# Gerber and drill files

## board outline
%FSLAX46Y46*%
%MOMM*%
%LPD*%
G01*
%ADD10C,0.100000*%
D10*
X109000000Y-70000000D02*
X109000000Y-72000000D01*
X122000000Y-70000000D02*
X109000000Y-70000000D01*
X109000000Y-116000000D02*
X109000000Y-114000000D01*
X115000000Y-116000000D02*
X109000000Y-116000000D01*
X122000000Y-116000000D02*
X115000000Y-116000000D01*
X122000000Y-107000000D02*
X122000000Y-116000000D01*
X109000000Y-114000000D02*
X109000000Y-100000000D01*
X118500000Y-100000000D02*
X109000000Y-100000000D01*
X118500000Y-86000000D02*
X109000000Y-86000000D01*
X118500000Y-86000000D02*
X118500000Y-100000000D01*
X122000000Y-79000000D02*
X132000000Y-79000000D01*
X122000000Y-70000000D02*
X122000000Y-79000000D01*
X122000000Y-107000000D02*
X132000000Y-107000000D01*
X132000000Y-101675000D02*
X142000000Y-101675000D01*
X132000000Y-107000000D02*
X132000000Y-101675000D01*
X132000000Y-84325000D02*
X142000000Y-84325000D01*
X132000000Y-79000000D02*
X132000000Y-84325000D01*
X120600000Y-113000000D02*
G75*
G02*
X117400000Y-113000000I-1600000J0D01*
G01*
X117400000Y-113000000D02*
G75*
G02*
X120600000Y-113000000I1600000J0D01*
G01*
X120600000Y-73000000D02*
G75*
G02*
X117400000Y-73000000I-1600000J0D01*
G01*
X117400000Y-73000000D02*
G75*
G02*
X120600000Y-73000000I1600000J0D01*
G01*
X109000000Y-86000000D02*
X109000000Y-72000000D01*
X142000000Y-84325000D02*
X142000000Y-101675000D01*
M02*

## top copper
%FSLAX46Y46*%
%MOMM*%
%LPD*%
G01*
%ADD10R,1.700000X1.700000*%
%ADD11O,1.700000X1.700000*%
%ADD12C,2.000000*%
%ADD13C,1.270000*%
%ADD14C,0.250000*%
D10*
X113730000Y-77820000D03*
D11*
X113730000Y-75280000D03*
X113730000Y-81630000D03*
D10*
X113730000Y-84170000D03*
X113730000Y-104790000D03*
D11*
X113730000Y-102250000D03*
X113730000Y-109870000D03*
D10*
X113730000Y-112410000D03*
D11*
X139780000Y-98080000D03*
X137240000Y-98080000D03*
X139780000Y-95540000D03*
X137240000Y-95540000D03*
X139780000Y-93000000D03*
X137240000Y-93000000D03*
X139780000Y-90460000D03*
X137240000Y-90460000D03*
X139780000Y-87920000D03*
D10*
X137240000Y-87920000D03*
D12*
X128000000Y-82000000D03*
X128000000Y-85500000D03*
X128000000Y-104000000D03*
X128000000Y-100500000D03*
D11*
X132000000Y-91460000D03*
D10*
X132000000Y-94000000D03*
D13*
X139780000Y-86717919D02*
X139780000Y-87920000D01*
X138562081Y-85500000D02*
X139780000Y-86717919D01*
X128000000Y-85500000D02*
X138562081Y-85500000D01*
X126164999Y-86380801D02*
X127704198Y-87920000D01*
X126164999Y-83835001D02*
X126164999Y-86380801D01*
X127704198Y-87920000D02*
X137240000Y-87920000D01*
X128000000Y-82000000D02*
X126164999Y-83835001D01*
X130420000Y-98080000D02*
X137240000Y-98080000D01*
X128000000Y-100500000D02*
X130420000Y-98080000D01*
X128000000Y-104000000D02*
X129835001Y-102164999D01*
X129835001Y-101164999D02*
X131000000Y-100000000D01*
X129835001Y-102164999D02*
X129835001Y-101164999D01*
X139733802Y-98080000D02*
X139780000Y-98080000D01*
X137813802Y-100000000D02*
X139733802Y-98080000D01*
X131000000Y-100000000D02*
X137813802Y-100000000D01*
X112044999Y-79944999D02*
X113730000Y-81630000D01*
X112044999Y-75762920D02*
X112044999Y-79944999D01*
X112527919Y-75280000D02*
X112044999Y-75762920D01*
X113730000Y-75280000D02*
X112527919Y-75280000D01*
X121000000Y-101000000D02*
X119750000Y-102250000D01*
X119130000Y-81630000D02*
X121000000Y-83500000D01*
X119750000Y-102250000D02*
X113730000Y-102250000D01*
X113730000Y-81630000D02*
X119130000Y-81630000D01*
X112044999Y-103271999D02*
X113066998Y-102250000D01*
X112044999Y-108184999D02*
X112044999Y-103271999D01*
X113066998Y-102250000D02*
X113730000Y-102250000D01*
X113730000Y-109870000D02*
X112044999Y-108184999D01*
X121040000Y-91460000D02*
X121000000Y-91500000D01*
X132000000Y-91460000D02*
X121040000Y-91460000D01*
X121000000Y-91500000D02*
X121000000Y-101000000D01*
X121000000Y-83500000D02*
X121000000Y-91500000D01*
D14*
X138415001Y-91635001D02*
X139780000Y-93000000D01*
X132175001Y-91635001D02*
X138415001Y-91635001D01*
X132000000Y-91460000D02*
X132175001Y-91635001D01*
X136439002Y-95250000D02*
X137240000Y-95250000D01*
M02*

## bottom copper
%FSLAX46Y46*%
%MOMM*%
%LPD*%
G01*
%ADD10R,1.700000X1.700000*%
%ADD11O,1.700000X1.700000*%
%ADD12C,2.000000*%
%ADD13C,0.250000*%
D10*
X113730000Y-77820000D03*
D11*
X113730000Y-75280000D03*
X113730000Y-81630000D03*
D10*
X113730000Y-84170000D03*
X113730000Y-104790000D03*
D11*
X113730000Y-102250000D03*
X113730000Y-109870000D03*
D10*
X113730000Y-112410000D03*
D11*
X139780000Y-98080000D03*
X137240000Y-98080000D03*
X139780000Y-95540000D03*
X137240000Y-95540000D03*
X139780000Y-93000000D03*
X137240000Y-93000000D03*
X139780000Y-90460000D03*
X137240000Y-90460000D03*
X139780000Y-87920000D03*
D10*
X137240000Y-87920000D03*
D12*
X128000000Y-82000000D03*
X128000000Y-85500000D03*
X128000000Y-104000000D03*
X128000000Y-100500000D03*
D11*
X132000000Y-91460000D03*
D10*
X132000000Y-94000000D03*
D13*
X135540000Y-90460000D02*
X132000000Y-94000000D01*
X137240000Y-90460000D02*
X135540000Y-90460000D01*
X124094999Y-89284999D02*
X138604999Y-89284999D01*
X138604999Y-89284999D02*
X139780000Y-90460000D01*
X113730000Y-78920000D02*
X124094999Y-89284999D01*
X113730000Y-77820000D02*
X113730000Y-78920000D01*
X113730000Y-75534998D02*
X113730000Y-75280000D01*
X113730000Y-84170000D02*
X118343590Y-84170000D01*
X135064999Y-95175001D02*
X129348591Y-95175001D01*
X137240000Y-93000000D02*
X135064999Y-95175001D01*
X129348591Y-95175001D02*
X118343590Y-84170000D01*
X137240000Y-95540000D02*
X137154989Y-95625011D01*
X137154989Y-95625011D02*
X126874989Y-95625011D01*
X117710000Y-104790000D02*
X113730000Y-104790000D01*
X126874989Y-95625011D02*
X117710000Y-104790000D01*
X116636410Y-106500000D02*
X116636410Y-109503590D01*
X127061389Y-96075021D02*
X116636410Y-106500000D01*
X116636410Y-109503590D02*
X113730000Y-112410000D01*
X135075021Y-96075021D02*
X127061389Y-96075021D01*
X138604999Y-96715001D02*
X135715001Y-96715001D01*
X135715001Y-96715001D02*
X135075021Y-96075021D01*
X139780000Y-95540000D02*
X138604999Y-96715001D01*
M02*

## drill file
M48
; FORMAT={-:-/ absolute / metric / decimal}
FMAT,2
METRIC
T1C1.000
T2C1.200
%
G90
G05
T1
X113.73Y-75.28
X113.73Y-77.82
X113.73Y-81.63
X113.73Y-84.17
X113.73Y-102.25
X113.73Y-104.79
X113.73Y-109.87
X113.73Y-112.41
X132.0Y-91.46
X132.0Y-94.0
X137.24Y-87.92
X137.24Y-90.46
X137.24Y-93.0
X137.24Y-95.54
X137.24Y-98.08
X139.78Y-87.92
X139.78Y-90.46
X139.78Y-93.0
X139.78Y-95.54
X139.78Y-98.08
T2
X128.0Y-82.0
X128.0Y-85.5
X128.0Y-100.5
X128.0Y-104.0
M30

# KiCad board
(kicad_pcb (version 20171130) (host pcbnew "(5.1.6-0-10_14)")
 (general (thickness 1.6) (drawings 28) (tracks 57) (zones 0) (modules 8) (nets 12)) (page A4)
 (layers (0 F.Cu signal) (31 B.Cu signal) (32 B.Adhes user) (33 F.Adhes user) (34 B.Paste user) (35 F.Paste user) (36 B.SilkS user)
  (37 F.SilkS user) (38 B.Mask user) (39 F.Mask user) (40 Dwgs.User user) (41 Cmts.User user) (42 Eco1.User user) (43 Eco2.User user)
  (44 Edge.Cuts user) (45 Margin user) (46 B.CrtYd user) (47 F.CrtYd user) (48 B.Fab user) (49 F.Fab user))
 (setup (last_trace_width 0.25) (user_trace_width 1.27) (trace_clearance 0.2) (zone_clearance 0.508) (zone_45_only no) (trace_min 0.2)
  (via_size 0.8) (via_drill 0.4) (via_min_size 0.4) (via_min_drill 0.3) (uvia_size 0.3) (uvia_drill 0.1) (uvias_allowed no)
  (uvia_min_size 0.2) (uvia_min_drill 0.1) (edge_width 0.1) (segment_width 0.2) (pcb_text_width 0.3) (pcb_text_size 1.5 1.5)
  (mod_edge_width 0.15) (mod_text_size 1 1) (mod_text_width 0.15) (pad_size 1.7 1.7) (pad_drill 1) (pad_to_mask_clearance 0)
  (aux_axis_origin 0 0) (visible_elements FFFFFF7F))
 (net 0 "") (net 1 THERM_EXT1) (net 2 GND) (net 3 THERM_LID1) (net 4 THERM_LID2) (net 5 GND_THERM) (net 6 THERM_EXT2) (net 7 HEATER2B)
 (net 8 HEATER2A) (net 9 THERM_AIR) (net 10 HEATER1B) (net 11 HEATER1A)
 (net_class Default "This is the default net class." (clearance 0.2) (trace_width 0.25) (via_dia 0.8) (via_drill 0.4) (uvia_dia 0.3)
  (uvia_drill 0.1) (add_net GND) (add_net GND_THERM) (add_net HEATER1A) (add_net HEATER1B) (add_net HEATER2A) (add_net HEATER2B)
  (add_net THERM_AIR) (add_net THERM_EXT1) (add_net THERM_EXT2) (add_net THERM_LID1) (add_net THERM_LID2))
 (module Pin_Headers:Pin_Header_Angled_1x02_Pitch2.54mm (layer F.Cu) (at 113.73 77.82 180)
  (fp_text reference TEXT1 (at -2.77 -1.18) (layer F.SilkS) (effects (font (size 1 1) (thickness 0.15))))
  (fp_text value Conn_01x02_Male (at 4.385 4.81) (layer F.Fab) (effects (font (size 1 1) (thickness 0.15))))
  (pad 1 thru_hole rect (at 0 0 180) (size 1.7 1.7) (drill 1) (layers *.Cu *.Mask) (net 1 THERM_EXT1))
  (pad 2 thru_hole oval (at 0 2.54 180) (size 1.7 1.7) (drill 1) (layers *.Cu *.Mask) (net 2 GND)))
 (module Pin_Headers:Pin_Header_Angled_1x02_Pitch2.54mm (layer F.Cu) (at 113.73 84.17 180)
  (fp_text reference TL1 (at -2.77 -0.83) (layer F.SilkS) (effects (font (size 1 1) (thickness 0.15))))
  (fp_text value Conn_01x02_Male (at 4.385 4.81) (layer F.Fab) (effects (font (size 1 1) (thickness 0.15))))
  (pad 2 thru_hole oval (at 0 2.54 180) (size 1.7 1.7) (drill 1) (layers *.Cu *.Mask) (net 2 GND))
  (pad 1 thru_hole rect (at 0 0 180) (size 1.7 1.7) (drill 1) (layers *.Cu *.Mask) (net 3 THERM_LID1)))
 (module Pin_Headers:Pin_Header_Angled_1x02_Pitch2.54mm (layer F.Cu) (at 113.73 104.79 180)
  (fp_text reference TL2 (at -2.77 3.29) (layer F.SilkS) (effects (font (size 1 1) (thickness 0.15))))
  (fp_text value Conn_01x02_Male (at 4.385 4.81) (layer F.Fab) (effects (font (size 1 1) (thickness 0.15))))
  (pad 1 thru_hole rect (at 0 0 180) (size 1.7 1.7) (drill 1) (layers *.Cu *.Mask) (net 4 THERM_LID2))
  (pad 2 thru_hole oval (at 0 2.54 180) (size 1.7 1.7) (drill 1) (layers *.Cu *.Mask) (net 2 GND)))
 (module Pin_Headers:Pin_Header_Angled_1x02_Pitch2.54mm (layer F.Cu) (at 113.73 112.41 180)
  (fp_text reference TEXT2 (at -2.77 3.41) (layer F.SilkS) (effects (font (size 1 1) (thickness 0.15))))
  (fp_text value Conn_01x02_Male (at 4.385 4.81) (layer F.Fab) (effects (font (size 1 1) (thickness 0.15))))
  (pad 2 thru_hole oval (at 0 2.54 180) (size 1.7 1.7) (drill 1) (layers *.Cu *.Mask) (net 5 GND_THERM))
  (pad 1 thru_hole rect (at 0 0 180) (size 1.7 1.7) (drill 1) (layers *.Cu *.Mask) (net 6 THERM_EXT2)))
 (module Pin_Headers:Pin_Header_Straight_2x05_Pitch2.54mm (layer F.Cu) (at 137.24 87.92)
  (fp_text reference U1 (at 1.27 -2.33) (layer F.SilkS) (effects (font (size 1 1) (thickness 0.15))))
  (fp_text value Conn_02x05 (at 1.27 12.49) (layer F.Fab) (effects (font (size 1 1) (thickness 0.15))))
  (pad 10 thru_hole oval (at 2.54 10.16) (size 1.7 1.7) (drill 1) (layers *.Cu *.Mask) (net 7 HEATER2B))
  (pad 9 thru_hole oval (at 0 10.16) (size 1.7 1.7) (drill 1) (layers *.Cu *.Mask) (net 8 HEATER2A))
  (pad 8 thru_hole oval (at 2.54 7.62) (size 1.7 1.7) (drill 1) (layers *.Cu *.Mask) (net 6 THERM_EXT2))
  (pad 7 thru_hole oval (at 0 7.62) (size 1.7 1.7) (drill 1) (layers *.Cu *.Mask) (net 4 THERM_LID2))
  (pad 6 thru_hole oval (at 2.54 5.08) (size 1.7 1.7) (drill 1) (layers *.Cu *.Mask) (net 2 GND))
  (pad 5 thru_hole oval (at 0 5.08) (size 1.7 1.7) (drill 1) (layers *.Cu *.Mask) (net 3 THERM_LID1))
  (pad 4 thru_hole oval (at 2.54 2.54) (size 1.7 1.7) (drill 1) (layers *.Cu *.Mask) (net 1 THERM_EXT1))
  (pad 3 thru_hole oval (at 0 2.54) (size 1.7 1.7) (drill 1) (layers *.Cu *.Mask) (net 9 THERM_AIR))
  (pad 2 thru_hole oval (at 2.54 0) (size 1.7 1.7) (drill 1) (layers *.Cu *.Mask) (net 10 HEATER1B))
  (pad 1 thru_hole rect (at 0 0) (size 1.7 1.7) (drill 1) (layers *.Cu *.Mask) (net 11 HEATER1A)))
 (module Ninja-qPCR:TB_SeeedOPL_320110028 (layer F.Cu) (at 128 82 270)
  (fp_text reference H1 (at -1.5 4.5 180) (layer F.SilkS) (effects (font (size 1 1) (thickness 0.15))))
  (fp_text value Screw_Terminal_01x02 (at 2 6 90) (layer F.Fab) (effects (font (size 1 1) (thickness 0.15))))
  (pad 1 thru_hole circle (at 0 0 270) (size 2 2) (drill 1.2) (layers *.Cu *.Mask) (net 11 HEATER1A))
  (pad 2 thru_hole circle (at 3.5 0 270) (size 2 2) (drill 1.2) (layers *.Cu *.Mask) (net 10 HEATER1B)))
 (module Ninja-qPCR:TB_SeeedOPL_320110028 (layer F.Cu) (at 128 100.5 270)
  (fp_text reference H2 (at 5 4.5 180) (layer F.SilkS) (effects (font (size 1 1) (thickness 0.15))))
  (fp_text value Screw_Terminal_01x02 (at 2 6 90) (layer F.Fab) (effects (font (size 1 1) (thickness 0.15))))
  (pad 2 thru_hole circle (at 3.5 0 270) (size 2 2) (drill 1.2) (layers *.Cu *.Mask) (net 7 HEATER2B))
  (pad 1 thru_hole circle (at 0 0 270) (size 2 2) (drill 1.2) (layers *.Cu *.Mask) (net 8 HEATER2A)))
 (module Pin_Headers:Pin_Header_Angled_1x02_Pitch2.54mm (layer F.Cu) (at 132 94 180)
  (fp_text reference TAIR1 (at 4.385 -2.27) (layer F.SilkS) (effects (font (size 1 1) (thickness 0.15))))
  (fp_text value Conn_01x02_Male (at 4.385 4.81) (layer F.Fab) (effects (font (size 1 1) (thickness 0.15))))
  (pad 2 thru_hole oval (at 0 2.54 180) (size 1.7 1.7) (drill 1) (layers *.Cu *.Mask) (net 2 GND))
  (pad 1 thru_hole rect (at 0 0 180) (size 1.7 1.7) (drill 1) (layers *.Cu *.Mask) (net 9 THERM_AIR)))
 (gr_line (start 109 70) (end 109 72) (layer Edge.Cuts) (width 0.1))
 (gr_line (start 122 70) (end 109 70) (layer Edge.Cuts) (width 0.1))
 (gr_line (start 109 116) (end 109 114) (layer Edge.Cuts) (width 0.1))
 (gr_line (start 115 116) (end 109 116) (layer Edge.Cuts) (width 0.1))
 (gr_line (start 122 116) (end 115 116) (layer Edge.Cuts) (width 0.1))
 (gr_line (start 122 107) (end 122 116) (layer Edge.Cuts) (width 0.1))
 (gr_line (start 109 114) (end 109 100) (layer Edge.Cuts) (width 0.1))
 (gr_line (start 118.5 100) (end 109 100) (layer Edge.Cuts) (width 0.1))
 (gr_line (start 118.5 86) (end 109 86) (layer Edge.Cuts) (width 0.1))
 (gr_line (start 118.5 86) (end 118.5 100) (layer Edge.Cuts) (width 0.1))
 (gr_line (start 122 79) (end 132 79) (layer Edge.Cuts) (width 0.1))
 (gr_line (start 122 70) (end 122 79) (layer Edge.Cuts) (width 0.1))
 (gr_line (start 122 107) (end 132 107) (layer Edge.Cuts) (width 0.1))
 (gr_line (start 132 101.675) (end 142 101.675) (layer Edge.Cuts) (width 0.1))
 (gr_line (start 132 107) (end 132 101.675) (layer Edge.Cuts) (width 0.1))
 (gr_line (start 132 84.325) (end 142 84.325) (layer Edge.Cuts) (width 0.1))
 (gr_line (start 132 79) (end 132 84.325) (layer Edge.Cuts) (width 0.1))
 (gr_circle (center 119 113) (end 120.6 113) (layer Edge.Cuts) (width 0.1))
 (gr_circle (center 119 73) (end 120.6 73) (layer Edge.Cuts) (width 0.1))
 (gr_line (start 109 86) (end 109 72) (layer Edge.Cuts) (width 0.1))
 (gr_line (start 142 84.325) (end 142 101.675) (layer Edge.Cuts) (width 0.1))
 (segment (start 139.78 86.717919) (end 139.78 87.92) (width 1.27) (layer F.Cu) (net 10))
 (segment (start 138.562081 85.5) (end 139.78 86.717919) (width 1.27) (layer F.Cu) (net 10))
 (segment (start 128 85.5) (end 138.562081 85.5) (width 1.27) (layer F.Cu) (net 10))
 (segment (start 126.164999 86.380801) (end 127.704198 87.92) (width 1.27) (layer F.Cu) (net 11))
 (segment (start 126.164999 83.835001) (end 126.164999 86.380801) (width 1.27) (layer F.Cu) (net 11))
 (segment (start 127.704198 87.92) (end 137.24 87.92) (width 1.27) (layer F.Cu) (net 11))
 (segment (start 128 82) (end 126.164999 83.835001) (width 1.27) (layer F.Cu) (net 11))
 (segment (start 130.42 98.08) (end 137.24 98.08) (width 1.27) (layer F.Cu) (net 8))
 (segment (start 128 100.5) (end 130.42 98.08) (width 1.27) (layer F.Cu) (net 8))
 (segment (start 128 104) (end 129.835001 102.164999) (width 1.27) (layer F.Cu) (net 7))
 (segment (start 129.835001 101.164999) (end 131 100) (width 1.27) (layer F.Cu) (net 7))
 (segment (start 129.835001 102.164999) (end 129.835001 101.164999) (width 1.27) (layer F.Cu) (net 7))
 (segment (start 139.733802 98.08) (end 139.78 98.08) (width 1.27) (layer F.Cu) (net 7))
 (segment (start 137.813802 100) (end 139.733802 98.08) (width 1.27) (layer F.Cu) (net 7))
 (segment (start 131 100) (end 137.813802 100) (width 1.27) (layer F.Cu) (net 7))
 (segment (start 135.54 90.46) (end 132 94) (width 0.25) (layer B.Cu) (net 9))
 (segment (start 137.24 90.46) (end 135.54 90.46) (width 0.25) (layer B.Cu) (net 9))
 (segment (start 124.094999 89.284999) (end 138.604999 89.284999) (width 0.25) (layer B.Cu) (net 1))
 (segment (start 138.604999 89.284999) (end 139.78 90.46) (width 0.25) (layer B.Cu) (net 1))
 (segment (start 113.73 78.92) (end 124.094999 89.284999) (width 0.25) (layer B.Cu) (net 1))
 (segment (start 113.73 77.82) (end 113.73 78.92) (width 0.25) (layer B.Cu) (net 1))
 (segment (start 113.73 75.534998) (end 113.73 75.28) (width 0.25) (layer B.Cu) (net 5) (status 30))
 (segment (start 112.044999 79.944999) (end 113.73 81.63) (width 1.27) (layer F.Cu) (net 5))
 (segment (start 112.044999 75.76292) (end 112.044999 79.944999) (width 1.27) (layer F.Cu) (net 5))
 (segment (start 112.527919 75.28) (end 112.044999 75.76292) (width 1.27) (layer F.Cu) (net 5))
 (segment (start 113.73 75.28) (end 112.527919 75.28) (width 1.27) (layer F.Cu) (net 5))
 (segment (start 121 101) (end 119.75 102.25) (width 1.27) (layer F.Cu) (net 5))
 (segment (start 119.13 81.63) (end 121 83.5) (width 1.27) (layer F.Cu) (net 5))
 (segment (start 119.75 102.25) (end 113.73 102.25) (width 1.27) (layer F.Cu) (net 5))
 (segment (start 113.73 81.63) (end 119.13 81.63) (width 1.27) (layer F.Cu) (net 5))
 (segment (start 112.044999 103.271999) (end 113.066998 102.25) (width 1.27) (layer F.Cu) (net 5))
 (segment (start 112.044999 108.184999) (end 112.044999 103.271999) (width 1.27) (layer F.Cu) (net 5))
 (segment (start 113.066998 102.25) (end 113.73 102.25) (width 1.27) (layer F.Cu) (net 5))
 (segment (start 113.73 109.87) (end 112.044999 108.184999) (width 1.27) (layer F.Cu) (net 5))
 (segment (start 121.04 91.46) (end 121 91.5) (width 1.27) (layer F.Cu) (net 5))
 (segment (start 132 91.46) (end 121.04 91.46) (width 1.27) (layer F.Cu) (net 5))
 (segment (start 121 91.5) (end 121 101) (width 1.27) (layer F.Cu) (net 5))
 (segment (start 121 83.5) (end 121 91.5) (width 1.27) (layer F.Cu) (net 5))
 (segment (start 138.415001 91.635001) (end 139.78 93) (width 0.25) (layer F.Cu) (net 5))
 (segment (start 132.175001 91.635001) (end 138.415001 91.635001) (width 0.25) (layer F.Cu) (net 5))
 (segment (start 132 91.46) (end 132.175001 91.635001) (width 0.25) (layer F.Cu) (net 5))
 (segment (start 113.73 84.17) (end 118.34359 84.17) (width 0.25) (layer B.Cu) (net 3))
 (segment (start 135.064999 95.175001) (end 129.348591 95.175001) (width 0.25) (layer B.Cu) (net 3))
 (segment (start 137.24 93) (end 135.064999 95.175001) (width 0.25) (layer B.Cu) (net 3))
 (segment (start 129.348591 95.175001) (end 118.34359 84.17) (width 0.25) (layer B.Cu) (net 3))
 (segment (start 136.439002 95.25) (end 137.24 95.25) (width 0.25) (layer F.Cu) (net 4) (status 20))
 (segment (start 137.24 95.54) (end 137.154989 95.625011) (width 0.25) (layer B.Cu) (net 4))
 (segment (start 137.154989 95.625011) (end 126.874989 95.625011) (width 0.25) (layer B.Cu) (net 4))
 (segment (start 117.71 104.79) (end 113.73 104.79) (width 0.25) (layer B.Cu) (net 4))
 (segment (start 126.874989 95.625011) (end 117.71 104.79) (width 0.25) (layer B.Cu) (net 4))
 (segment (start 116.63641 106.5) (end 116.63641 109.50359) (width 0.25) (layer B.Cu) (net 6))
 (segment (start 127.061389 96.075021) (end 116.63641 106.5) (width 0.25) (layer B.Cu) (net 6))
 (segment (start 116.63641 109.50359) (end 113.73 112.41) (width 0.25) (layer B.Cu) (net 6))
 (segment (start 135.075021 96.075021) (end 127.061389 96.075021) (width 0.25) (layer B.Cu) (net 6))
 (segment (start 138.604999 96.715001) (end 135.715001 96.715001) (width 0.25) (layer B.Cu) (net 6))
 (segment (start 135.715001 96.715001) (end 135.075021 96.075021) (width 0.25) (layer B.Cu) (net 6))
 (segment (start 139.78 95.54) (end 138.604999 96.715001) (width 0.25) (layer B.Cu) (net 6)))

